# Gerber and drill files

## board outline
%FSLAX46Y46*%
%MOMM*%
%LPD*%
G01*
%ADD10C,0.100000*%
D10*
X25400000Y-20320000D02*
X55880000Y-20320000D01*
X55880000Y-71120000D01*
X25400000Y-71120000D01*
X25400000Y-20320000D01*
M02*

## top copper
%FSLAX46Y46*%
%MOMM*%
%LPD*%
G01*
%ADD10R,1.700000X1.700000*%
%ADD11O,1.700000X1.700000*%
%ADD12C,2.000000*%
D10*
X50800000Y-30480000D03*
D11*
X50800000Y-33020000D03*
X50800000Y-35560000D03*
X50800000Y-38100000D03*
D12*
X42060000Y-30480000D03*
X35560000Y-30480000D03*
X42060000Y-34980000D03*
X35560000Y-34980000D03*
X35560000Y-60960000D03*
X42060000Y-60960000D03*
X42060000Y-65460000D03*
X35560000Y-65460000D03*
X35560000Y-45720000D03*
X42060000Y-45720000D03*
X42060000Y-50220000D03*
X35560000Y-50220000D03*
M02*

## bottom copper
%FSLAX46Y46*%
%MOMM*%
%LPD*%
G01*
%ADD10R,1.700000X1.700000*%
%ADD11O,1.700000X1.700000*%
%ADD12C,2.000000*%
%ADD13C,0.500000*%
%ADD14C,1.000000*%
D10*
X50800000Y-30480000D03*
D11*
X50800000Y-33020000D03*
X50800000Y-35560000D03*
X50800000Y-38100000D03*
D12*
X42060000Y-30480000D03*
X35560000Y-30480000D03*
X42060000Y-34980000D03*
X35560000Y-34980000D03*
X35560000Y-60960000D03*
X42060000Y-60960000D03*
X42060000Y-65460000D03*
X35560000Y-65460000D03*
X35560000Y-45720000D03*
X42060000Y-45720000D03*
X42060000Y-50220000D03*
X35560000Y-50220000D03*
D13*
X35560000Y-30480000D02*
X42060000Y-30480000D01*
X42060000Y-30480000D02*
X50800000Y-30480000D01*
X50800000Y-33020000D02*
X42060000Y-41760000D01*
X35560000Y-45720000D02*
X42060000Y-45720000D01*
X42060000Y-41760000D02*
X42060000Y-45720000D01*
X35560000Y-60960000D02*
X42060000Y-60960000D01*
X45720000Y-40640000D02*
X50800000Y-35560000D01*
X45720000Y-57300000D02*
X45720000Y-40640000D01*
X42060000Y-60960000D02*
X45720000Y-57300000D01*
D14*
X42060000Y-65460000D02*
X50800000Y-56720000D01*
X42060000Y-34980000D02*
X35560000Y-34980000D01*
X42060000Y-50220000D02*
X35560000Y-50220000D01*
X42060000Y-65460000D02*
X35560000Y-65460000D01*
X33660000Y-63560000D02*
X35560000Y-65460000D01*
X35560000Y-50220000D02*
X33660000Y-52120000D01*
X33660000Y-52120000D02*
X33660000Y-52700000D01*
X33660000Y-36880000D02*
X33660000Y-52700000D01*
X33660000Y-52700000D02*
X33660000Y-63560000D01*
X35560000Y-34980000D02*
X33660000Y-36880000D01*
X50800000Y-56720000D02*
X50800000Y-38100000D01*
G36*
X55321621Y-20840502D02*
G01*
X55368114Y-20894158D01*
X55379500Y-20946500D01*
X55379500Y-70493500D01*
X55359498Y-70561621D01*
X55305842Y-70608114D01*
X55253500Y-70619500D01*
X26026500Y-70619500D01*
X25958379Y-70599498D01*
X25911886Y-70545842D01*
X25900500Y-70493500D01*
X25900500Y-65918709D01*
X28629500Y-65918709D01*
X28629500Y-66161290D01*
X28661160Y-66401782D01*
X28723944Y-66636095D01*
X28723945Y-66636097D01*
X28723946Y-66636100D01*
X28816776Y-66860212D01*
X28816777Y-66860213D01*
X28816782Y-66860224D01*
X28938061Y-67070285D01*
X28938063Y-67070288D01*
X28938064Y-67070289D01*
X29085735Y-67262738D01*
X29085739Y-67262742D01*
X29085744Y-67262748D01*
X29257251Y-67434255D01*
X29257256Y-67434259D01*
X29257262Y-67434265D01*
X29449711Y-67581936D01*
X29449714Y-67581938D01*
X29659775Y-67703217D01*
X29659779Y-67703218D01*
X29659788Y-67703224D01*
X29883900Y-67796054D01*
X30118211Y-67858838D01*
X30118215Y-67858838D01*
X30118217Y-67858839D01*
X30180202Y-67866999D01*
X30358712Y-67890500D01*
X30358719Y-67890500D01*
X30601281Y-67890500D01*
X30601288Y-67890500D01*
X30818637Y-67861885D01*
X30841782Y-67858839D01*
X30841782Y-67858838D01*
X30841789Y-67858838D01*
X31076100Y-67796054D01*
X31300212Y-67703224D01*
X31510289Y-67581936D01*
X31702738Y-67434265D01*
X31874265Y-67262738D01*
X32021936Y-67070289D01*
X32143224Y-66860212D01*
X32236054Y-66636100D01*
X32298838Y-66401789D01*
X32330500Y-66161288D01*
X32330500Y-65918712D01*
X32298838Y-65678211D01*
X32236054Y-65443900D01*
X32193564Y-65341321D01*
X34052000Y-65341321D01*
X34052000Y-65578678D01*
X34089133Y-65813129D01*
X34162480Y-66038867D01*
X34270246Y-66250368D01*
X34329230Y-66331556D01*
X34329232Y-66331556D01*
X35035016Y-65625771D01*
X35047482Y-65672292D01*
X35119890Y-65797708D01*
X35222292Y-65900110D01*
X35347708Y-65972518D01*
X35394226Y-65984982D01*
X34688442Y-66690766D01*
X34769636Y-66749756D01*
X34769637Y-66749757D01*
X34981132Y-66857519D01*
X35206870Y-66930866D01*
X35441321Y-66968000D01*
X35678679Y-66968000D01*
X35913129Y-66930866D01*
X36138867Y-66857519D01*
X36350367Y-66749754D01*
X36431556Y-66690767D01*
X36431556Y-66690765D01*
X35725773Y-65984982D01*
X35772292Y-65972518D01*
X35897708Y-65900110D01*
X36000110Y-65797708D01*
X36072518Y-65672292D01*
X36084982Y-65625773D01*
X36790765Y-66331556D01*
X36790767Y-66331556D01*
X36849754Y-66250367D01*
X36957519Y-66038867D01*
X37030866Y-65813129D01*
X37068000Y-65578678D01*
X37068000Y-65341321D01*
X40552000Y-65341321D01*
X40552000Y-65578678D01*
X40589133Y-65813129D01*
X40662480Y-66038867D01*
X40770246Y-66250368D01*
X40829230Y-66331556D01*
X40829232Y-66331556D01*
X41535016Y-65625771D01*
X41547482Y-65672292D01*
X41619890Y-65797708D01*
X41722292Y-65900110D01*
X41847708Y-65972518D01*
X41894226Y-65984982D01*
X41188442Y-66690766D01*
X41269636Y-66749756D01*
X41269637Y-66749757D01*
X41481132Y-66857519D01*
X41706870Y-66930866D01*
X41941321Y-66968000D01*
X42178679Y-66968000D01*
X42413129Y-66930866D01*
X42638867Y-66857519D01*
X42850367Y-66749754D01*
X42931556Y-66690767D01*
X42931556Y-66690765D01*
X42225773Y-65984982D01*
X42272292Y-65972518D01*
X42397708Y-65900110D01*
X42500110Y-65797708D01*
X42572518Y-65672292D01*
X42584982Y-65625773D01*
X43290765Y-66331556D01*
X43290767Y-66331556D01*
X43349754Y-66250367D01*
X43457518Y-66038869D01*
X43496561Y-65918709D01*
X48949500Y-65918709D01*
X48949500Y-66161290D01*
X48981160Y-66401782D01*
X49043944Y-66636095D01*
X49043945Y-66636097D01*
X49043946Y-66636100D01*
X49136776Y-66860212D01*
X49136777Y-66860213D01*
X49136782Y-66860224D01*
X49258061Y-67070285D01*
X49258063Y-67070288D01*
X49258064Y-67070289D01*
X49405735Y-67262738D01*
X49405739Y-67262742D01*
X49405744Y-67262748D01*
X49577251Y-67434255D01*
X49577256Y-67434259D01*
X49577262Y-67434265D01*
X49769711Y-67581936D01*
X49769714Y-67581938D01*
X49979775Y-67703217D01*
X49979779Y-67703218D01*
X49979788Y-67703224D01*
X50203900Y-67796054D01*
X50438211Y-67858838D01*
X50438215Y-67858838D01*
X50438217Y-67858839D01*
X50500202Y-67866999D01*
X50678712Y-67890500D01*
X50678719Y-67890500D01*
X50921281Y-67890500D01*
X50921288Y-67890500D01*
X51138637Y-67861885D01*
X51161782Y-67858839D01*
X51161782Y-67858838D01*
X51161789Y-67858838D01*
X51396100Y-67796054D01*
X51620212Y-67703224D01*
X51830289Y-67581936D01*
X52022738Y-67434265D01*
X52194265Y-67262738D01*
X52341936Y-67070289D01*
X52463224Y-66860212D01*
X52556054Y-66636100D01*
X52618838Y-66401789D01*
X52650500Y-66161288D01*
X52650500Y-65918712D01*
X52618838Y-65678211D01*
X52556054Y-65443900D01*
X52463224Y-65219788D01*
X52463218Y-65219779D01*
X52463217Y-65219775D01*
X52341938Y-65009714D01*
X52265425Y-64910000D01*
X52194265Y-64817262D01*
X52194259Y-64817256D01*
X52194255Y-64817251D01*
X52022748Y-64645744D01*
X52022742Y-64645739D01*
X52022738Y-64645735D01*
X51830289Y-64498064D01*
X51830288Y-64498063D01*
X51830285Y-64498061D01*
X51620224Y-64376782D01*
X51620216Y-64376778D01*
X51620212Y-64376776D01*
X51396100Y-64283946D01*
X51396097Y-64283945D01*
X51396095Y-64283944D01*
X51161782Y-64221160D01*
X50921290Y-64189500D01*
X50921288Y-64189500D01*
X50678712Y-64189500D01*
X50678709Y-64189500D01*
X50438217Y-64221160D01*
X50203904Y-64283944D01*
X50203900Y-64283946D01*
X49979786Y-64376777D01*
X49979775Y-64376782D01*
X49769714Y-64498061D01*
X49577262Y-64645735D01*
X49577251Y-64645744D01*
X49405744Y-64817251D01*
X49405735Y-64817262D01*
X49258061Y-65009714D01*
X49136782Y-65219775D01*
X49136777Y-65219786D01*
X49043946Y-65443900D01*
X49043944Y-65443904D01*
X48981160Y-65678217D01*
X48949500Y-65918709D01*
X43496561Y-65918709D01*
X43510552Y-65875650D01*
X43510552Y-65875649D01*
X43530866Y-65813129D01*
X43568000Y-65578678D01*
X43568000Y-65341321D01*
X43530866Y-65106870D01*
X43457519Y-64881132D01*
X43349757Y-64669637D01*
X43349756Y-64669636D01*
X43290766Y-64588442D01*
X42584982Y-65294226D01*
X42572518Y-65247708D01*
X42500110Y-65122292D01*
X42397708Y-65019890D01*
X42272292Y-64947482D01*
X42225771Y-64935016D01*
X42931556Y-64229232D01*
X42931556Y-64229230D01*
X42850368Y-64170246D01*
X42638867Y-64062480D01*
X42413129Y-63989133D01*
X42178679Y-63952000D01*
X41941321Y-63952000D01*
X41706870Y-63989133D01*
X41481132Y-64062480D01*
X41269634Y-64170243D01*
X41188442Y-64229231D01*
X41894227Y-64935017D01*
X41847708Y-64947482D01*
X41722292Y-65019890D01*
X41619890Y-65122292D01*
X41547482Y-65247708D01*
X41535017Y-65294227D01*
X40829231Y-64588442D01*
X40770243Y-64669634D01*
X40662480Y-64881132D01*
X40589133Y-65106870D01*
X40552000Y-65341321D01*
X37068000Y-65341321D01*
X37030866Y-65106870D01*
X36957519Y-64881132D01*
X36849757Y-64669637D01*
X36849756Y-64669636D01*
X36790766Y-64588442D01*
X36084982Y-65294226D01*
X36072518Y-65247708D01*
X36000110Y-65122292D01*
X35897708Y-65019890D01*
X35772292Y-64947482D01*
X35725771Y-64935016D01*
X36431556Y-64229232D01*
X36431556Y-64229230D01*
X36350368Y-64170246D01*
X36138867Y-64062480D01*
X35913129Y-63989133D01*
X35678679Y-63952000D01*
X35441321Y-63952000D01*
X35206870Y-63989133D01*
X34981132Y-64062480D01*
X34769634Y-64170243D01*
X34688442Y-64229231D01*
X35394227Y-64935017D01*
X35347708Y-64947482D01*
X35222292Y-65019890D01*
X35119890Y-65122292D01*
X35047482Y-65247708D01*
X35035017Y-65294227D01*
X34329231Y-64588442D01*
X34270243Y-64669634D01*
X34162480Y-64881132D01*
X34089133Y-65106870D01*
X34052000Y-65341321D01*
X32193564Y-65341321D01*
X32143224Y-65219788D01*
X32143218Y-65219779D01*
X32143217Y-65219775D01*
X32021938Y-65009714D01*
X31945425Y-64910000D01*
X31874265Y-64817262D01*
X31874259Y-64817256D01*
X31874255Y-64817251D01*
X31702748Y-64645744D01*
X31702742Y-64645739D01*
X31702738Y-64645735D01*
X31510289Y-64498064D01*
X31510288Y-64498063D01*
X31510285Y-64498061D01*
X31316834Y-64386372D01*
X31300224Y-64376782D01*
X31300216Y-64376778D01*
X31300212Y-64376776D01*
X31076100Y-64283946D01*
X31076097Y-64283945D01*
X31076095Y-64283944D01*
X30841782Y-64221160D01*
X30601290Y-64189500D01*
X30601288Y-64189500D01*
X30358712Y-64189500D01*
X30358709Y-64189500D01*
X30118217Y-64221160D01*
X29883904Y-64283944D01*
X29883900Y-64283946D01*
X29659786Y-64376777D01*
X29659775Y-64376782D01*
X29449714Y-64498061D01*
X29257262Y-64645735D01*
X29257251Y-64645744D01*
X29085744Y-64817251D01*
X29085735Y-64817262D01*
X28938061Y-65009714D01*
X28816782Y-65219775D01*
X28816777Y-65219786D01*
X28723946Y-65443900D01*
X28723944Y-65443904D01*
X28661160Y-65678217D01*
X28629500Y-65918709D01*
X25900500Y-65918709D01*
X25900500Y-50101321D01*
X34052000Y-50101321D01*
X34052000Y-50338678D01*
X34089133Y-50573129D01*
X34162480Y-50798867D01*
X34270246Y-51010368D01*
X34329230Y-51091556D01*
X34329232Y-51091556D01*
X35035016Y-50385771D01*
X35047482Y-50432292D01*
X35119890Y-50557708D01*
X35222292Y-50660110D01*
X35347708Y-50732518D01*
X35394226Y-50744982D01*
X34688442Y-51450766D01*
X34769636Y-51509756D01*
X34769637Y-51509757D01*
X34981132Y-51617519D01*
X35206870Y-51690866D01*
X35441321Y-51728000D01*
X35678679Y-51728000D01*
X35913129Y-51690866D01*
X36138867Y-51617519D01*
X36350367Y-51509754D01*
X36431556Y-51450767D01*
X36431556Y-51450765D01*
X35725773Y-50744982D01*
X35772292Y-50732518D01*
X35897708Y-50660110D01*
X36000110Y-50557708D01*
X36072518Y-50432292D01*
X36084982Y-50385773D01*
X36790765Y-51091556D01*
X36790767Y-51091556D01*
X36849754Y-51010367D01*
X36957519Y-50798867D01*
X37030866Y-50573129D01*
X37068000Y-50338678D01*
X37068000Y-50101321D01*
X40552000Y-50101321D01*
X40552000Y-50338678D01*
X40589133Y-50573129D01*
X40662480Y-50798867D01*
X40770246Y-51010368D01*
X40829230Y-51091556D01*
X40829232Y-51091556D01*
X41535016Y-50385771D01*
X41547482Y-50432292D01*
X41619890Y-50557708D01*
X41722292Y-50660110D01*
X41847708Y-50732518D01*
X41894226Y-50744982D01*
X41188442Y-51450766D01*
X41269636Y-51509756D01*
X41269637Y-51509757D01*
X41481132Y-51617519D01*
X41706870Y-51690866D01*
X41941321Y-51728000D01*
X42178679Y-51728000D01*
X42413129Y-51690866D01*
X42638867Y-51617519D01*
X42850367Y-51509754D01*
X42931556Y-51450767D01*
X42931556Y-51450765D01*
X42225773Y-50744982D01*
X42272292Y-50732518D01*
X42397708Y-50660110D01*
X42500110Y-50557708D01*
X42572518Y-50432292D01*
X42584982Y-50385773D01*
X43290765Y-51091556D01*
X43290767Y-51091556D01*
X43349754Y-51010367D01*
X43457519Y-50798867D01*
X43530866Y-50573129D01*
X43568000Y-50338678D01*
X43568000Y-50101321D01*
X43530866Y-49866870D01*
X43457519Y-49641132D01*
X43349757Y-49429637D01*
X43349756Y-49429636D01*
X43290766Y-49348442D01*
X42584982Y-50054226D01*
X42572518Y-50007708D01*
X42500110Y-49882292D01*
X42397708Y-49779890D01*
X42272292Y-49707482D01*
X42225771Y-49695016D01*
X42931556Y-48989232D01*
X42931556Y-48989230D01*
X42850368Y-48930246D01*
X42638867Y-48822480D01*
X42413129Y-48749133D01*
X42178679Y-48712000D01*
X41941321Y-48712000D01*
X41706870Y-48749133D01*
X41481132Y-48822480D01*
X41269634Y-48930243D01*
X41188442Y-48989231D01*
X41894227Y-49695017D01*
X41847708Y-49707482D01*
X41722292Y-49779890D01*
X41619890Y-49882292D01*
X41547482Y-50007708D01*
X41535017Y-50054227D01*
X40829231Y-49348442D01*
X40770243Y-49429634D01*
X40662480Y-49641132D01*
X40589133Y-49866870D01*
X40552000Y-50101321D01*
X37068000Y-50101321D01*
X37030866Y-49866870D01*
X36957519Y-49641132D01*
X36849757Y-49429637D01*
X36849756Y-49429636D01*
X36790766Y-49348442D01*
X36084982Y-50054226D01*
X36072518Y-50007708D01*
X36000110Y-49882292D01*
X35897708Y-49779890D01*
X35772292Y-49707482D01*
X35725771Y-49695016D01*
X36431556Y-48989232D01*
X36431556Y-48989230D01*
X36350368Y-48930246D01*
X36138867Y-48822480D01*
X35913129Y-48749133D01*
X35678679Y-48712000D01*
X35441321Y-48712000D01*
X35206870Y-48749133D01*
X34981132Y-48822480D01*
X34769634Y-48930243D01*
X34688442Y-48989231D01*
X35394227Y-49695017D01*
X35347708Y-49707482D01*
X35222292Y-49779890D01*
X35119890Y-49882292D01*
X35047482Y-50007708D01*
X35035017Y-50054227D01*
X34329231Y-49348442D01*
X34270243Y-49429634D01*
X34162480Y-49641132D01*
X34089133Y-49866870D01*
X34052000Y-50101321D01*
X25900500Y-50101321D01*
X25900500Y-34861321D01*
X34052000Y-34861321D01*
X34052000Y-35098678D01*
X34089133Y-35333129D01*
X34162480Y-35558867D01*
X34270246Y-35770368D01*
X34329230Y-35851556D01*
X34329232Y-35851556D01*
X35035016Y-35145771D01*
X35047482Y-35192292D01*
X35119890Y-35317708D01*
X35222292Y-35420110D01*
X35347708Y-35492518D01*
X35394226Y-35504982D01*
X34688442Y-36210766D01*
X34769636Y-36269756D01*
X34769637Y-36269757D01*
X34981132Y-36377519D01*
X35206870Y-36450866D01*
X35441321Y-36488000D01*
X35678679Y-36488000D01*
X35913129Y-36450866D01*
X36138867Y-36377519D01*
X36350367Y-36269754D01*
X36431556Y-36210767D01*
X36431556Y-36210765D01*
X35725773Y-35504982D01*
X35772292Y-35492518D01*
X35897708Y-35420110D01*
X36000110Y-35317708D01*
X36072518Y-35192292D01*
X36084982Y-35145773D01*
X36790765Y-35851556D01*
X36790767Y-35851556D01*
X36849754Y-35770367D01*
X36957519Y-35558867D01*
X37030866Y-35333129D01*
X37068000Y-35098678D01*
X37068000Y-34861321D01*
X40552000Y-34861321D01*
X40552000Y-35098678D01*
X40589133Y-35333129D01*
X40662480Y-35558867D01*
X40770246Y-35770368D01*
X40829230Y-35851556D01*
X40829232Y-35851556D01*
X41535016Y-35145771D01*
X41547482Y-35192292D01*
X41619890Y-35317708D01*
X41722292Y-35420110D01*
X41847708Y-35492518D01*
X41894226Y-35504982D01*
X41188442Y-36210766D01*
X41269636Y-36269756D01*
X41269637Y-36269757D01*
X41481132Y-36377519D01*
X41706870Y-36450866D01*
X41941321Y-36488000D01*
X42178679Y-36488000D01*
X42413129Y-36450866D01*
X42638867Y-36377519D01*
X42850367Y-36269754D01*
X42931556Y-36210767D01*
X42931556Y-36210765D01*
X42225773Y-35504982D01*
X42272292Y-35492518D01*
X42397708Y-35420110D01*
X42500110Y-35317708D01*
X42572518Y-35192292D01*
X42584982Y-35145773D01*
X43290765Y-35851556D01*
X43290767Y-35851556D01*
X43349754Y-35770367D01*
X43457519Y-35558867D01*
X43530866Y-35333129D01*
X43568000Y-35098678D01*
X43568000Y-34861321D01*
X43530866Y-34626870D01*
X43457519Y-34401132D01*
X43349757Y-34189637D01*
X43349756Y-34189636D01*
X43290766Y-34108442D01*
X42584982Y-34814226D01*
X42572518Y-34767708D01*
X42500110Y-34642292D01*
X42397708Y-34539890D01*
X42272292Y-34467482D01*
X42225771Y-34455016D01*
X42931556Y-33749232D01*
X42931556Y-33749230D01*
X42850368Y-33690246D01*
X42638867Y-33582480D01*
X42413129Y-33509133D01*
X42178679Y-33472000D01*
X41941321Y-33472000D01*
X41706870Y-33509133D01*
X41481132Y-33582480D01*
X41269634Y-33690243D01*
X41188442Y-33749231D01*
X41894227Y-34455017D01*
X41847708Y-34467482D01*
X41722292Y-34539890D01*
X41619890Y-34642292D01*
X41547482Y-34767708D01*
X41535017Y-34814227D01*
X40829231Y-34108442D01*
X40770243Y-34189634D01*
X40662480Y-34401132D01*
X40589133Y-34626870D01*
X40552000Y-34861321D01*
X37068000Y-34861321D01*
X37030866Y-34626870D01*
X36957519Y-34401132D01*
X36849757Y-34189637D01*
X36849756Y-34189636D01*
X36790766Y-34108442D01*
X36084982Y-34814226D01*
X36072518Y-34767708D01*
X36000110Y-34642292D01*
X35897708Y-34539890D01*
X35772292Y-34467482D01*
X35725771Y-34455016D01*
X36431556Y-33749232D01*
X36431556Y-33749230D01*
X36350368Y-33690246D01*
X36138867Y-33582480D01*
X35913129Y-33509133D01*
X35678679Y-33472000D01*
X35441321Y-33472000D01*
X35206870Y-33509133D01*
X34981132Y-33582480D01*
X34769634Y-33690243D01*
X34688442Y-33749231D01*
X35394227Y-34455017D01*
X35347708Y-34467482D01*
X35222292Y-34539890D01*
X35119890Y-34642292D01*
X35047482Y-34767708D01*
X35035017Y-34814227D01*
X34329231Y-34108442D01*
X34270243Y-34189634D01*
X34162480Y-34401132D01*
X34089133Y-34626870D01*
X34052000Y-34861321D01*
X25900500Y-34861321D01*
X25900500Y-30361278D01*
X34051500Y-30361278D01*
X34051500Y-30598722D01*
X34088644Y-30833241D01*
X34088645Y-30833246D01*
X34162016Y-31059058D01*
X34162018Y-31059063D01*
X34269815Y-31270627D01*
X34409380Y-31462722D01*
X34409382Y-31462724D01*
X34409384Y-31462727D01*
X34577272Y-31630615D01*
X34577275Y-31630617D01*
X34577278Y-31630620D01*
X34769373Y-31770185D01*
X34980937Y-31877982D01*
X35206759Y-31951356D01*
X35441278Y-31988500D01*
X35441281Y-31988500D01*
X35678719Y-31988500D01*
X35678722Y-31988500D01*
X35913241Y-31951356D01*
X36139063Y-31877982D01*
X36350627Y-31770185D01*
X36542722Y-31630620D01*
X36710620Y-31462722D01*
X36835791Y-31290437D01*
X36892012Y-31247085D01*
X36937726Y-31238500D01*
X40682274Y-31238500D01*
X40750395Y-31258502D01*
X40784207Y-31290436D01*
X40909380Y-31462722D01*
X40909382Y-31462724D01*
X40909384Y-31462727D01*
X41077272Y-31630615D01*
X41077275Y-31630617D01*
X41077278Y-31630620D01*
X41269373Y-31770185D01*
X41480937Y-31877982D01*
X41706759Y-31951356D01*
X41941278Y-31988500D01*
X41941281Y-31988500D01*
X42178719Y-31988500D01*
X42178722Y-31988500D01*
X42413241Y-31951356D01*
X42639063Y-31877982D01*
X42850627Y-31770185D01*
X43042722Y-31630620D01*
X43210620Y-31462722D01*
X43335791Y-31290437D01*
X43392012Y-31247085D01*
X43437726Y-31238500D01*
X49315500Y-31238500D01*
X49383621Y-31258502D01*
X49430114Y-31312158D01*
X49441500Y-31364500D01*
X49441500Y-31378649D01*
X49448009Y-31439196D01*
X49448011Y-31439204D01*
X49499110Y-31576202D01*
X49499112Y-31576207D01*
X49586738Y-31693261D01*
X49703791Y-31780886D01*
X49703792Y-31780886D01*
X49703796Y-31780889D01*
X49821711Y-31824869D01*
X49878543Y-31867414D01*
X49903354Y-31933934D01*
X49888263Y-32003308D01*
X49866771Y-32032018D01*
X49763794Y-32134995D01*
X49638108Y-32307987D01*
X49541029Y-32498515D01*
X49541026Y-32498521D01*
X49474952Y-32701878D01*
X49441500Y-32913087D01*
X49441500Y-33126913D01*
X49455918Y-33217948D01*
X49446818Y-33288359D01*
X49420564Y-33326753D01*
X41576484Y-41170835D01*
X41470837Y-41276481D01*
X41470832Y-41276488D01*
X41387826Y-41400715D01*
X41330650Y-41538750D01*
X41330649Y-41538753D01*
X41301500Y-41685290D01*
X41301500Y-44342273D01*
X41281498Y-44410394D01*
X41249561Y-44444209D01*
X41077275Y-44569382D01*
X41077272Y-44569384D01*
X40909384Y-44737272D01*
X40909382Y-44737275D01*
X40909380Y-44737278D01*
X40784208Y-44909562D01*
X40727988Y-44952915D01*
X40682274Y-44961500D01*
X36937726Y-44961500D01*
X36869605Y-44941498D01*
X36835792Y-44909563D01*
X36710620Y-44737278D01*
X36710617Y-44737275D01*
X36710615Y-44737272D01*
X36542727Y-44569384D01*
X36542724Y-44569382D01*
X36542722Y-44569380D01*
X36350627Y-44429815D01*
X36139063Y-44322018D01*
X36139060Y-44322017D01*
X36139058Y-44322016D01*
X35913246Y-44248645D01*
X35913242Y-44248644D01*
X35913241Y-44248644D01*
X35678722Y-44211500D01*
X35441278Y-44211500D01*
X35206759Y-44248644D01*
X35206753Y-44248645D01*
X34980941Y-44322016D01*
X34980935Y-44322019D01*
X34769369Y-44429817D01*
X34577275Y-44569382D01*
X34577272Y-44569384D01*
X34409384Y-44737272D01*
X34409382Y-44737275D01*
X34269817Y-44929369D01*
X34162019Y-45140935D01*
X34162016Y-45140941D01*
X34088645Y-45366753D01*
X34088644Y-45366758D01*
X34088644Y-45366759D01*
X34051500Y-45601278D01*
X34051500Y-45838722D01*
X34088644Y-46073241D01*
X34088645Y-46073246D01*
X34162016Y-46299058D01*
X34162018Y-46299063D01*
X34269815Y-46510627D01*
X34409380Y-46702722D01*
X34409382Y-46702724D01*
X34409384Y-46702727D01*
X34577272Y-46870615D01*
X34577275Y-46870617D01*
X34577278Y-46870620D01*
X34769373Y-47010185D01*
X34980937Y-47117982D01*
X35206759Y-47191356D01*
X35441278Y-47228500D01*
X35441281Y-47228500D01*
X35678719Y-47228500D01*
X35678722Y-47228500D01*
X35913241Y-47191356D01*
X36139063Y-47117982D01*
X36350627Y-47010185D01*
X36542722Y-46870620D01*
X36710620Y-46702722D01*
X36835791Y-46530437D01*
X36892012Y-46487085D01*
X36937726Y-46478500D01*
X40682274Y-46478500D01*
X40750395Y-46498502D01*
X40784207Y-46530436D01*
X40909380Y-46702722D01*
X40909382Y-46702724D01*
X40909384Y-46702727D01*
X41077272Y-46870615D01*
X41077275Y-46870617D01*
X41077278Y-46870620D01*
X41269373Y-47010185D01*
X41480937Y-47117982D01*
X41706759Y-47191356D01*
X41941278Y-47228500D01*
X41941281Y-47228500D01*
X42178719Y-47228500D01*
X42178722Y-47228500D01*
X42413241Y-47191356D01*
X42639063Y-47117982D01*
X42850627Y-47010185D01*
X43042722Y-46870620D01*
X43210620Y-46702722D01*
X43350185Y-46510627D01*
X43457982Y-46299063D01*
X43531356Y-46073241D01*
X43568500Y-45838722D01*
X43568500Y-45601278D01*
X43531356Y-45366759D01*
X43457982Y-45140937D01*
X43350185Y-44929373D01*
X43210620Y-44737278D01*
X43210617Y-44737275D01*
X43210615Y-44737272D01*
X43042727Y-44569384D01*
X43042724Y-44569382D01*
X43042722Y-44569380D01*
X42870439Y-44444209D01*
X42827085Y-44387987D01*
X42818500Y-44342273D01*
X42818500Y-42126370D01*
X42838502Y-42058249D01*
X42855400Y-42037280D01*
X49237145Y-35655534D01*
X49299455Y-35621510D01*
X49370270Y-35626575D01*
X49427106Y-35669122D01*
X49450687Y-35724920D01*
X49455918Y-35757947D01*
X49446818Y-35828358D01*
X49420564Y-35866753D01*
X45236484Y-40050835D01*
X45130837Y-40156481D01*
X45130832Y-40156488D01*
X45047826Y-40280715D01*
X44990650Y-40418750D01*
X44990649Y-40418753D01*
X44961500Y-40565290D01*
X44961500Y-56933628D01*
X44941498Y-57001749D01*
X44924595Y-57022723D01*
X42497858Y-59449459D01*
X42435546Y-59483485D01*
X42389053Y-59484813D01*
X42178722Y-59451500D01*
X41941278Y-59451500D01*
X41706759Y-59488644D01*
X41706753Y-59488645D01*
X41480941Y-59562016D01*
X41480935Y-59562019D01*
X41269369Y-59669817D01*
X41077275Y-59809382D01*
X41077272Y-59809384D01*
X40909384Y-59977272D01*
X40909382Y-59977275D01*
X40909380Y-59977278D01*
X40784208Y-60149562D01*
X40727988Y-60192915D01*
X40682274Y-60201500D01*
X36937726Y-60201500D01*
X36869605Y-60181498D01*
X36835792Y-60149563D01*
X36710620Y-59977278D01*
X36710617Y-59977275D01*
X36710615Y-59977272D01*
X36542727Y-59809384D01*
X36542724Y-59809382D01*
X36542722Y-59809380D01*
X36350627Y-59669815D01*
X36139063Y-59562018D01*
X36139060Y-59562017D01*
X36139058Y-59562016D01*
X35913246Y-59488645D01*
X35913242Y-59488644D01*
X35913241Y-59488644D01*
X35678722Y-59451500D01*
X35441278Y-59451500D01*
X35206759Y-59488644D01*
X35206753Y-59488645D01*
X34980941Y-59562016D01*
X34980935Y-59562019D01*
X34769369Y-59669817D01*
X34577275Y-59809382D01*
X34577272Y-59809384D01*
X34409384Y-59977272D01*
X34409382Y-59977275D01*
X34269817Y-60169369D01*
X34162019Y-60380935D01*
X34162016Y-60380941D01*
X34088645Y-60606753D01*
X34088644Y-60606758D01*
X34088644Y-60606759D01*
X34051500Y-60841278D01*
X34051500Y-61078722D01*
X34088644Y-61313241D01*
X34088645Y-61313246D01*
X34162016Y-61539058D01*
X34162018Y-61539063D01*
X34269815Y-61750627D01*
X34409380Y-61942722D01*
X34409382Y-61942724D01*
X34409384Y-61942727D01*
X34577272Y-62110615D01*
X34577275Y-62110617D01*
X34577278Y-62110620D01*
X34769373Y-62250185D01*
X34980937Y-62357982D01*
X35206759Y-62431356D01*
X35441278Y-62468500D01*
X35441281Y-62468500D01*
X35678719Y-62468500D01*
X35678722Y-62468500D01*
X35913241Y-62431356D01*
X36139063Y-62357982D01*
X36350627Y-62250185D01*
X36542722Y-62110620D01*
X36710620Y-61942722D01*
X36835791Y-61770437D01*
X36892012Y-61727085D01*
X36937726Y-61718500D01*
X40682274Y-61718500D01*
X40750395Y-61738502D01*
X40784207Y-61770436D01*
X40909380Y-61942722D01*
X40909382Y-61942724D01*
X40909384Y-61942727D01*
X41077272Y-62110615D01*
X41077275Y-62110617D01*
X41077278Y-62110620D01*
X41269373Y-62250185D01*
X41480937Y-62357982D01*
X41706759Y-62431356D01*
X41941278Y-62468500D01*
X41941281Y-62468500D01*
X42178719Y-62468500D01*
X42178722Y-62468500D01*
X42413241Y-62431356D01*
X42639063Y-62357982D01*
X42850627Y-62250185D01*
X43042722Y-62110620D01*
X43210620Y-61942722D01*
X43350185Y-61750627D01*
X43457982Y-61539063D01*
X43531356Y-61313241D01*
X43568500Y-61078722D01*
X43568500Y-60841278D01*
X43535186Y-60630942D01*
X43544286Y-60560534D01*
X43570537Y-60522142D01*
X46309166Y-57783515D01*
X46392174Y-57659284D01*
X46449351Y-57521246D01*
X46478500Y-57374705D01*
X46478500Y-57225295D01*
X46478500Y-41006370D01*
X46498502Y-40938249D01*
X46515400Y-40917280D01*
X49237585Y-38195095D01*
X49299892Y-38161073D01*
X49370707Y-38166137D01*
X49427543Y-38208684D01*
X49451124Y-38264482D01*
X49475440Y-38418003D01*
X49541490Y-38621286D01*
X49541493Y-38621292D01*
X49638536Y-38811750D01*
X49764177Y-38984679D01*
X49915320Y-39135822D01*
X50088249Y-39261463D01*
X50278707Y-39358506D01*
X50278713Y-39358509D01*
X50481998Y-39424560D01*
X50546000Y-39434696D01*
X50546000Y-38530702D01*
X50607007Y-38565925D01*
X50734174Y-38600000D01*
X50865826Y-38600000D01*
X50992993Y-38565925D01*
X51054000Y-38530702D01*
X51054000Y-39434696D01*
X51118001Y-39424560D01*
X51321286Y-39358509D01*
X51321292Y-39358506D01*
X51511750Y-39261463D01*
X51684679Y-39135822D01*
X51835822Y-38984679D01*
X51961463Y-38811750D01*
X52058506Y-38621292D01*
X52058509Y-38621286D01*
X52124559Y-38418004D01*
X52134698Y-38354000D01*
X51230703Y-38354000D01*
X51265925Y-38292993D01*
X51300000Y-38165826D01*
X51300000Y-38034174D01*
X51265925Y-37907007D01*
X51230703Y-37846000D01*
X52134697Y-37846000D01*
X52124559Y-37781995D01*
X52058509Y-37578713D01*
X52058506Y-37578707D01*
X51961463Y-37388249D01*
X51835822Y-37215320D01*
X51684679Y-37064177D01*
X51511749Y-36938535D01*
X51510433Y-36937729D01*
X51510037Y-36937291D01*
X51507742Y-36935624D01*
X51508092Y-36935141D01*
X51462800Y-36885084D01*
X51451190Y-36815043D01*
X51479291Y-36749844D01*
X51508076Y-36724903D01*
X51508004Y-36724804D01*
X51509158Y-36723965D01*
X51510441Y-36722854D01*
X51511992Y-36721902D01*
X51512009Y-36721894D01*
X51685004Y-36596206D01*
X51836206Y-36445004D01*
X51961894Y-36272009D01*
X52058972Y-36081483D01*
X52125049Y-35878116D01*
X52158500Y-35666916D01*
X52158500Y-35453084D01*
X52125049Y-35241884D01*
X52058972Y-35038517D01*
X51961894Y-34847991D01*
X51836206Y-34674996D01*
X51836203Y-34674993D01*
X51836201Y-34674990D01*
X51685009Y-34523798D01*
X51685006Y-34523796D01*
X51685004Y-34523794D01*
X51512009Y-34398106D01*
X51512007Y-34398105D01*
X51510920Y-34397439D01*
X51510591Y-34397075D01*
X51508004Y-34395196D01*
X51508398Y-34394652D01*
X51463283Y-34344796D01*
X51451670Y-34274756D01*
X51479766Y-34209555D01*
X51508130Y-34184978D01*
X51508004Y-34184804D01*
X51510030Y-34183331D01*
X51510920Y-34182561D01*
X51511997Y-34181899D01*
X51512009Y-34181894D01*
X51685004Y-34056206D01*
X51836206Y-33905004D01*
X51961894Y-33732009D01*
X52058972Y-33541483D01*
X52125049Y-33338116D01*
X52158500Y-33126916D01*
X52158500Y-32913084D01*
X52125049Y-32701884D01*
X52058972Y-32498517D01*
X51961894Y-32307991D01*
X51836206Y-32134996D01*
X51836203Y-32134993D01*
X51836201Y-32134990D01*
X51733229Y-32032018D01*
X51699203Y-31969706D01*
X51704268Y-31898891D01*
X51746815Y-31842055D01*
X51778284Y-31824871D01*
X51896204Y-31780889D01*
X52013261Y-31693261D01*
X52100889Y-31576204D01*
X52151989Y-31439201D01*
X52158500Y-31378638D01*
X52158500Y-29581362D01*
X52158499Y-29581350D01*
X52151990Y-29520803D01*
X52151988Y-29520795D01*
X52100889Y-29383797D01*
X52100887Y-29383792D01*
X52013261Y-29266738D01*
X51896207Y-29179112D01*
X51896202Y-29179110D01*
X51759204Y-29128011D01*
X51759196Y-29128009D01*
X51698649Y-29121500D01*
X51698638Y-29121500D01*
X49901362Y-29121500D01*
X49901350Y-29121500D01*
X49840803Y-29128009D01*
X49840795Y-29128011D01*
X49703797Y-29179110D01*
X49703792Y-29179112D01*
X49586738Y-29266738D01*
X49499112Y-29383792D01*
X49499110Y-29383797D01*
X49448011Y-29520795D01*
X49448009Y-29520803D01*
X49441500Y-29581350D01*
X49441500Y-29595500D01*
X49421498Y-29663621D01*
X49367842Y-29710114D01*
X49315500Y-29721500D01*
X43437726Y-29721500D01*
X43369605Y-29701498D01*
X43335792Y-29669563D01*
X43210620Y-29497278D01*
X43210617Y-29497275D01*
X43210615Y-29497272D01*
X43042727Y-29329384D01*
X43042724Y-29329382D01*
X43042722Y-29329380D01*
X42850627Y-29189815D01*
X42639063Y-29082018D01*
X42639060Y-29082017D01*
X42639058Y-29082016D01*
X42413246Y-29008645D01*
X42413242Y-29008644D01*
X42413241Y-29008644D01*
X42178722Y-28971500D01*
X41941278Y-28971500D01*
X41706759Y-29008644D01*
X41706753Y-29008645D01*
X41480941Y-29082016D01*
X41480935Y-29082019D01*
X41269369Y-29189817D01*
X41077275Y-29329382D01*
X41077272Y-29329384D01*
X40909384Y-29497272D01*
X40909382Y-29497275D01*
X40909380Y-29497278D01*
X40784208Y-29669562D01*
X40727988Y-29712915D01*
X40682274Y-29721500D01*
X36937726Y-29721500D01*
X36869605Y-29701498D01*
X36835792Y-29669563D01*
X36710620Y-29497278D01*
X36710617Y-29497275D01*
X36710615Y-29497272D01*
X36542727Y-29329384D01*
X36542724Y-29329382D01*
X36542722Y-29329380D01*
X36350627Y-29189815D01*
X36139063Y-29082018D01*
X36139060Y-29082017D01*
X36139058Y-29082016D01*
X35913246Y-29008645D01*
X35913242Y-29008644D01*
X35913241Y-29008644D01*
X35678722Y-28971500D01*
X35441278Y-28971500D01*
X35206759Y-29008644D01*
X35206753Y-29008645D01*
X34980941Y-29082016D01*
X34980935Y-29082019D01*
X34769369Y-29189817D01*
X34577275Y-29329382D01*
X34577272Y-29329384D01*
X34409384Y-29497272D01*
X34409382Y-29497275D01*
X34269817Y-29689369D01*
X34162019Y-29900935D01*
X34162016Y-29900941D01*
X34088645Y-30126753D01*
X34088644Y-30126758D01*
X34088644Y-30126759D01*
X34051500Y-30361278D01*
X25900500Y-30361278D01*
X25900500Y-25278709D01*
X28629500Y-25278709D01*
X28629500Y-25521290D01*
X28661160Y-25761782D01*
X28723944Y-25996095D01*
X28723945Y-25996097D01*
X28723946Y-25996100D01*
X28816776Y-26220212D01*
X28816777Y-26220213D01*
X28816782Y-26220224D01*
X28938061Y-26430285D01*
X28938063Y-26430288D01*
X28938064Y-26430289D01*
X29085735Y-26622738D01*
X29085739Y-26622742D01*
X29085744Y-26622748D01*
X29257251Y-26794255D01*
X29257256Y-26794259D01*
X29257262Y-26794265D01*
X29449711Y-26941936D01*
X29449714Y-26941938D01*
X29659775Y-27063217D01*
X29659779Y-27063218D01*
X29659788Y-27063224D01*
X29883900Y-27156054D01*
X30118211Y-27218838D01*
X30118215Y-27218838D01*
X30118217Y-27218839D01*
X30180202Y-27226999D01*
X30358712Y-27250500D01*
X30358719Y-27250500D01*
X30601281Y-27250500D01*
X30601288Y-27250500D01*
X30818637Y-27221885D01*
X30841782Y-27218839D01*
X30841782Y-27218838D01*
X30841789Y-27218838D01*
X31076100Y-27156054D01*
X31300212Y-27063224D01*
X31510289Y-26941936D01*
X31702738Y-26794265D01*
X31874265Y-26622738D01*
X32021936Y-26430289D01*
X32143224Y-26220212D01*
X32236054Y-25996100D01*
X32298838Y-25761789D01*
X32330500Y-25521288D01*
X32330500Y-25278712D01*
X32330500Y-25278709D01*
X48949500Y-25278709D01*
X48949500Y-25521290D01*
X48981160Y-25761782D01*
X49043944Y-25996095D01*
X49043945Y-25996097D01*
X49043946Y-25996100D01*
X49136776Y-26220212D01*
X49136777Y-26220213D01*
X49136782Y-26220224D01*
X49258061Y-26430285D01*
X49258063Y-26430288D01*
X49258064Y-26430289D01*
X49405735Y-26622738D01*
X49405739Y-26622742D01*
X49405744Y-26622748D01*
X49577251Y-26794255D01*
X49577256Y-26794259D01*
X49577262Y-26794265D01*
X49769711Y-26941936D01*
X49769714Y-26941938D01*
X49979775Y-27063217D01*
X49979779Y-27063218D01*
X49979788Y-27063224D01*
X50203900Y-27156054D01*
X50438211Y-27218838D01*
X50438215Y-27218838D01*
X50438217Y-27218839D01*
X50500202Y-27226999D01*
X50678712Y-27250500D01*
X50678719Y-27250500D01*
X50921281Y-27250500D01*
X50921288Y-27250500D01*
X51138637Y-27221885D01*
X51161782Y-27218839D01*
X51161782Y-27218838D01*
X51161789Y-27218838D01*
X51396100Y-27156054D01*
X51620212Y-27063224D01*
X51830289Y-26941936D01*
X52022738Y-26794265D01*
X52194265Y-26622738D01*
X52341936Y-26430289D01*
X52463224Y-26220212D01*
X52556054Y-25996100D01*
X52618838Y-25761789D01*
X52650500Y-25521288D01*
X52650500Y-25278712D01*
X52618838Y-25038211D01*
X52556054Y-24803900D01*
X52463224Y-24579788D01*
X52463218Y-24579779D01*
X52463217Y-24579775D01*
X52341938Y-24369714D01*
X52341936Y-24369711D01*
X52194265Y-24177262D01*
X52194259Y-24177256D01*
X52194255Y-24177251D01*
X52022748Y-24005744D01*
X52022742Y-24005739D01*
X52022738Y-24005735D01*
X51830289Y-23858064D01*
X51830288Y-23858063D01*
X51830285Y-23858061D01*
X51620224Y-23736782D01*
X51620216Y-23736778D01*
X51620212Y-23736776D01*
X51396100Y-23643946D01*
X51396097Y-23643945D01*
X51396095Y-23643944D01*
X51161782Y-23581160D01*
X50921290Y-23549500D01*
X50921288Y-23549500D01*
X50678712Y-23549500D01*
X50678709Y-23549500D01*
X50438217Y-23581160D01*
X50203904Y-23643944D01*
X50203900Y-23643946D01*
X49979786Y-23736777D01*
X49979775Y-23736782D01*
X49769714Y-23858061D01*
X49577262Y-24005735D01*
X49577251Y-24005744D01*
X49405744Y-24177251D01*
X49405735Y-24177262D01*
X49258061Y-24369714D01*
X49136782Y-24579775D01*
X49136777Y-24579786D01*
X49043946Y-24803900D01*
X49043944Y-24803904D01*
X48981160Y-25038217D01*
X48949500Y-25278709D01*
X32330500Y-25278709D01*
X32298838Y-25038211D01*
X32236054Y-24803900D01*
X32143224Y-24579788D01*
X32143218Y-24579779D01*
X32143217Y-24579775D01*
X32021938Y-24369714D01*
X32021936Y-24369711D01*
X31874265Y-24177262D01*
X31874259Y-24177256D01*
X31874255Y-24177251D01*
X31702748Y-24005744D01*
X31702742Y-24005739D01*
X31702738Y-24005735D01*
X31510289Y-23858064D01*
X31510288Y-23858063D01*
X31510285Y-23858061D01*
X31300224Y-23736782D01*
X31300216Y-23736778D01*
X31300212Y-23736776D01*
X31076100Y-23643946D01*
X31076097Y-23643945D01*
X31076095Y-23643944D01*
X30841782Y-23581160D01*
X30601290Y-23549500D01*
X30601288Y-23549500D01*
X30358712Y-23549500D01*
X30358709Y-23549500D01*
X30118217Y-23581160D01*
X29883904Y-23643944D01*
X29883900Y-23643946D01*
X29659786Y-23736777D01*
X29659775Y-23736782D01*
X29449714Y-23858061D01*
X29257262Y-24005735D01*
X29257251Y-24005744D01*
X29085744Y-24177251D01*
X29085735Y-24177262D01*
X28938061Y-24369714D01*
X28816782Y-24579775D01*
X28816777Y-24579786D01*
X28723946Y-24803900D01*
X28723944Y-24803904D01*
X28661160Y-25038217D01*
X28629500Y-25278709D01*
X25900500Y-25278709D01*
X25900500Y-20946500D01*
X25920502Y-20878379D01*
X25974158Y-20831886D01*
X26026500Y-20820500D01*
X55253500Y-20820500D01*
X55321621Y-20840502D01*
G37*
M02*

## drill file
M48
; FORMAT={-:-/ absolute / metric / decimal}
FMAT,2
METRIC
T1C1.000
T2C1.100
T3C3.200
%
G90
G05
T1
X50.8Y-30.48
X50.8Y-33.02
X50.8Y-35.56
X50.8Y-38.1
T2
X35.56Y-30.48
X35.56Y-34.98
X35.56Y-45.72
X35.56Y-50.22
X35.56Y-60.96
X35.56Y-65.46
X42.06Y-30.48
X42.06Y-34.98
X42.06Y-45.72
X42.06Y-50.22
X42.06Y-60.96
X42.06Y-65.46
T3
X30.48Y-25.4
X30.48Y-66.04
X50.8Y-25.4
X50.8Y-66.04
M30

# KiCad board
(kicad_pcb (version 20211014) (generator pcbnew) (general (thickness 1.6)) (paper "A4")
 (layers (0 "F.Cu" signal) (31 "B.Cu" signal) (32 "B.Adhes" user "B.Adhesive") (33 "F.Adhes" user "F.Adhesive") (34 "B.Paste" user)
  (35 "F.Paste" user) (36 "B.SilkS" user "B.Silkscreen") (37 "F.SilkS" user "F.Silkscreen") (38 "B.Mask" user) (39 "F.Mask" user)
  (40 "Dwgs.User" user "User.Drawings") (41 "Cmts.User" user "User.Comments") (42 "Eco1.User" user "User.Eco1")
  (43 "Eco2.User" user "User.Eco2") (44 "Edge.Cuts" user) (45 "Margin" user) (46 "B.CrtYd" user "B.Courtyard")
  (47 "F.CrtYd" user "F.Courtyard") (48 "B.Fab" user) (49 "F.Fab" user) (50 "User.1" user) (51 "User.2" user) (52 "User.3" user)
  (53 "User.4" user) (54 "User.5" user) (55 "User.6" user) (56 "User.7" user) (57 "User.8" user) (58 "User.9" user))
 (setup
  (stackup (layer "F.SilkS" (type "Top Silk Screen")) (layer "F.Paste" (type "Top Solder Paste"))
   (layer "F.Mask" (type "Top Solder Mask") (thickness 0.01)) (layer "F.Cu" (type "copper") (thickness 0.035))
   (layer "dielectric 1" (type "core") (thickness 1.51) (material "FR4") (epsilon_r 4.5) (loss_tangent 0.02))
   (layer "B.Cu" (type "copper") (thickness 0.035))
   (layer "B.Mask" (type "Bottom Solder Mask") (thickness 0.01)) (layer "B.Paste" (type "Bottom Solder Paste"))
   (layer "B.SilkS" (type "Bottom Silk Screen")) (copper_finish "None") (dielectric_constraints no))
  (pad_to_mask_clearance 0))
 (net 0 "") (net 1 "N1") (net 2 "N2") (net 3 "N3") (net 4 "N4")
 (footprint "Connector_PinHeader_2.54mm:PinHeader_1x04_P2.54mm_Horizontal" (layer "F.Cu") (at 50.8 30.48)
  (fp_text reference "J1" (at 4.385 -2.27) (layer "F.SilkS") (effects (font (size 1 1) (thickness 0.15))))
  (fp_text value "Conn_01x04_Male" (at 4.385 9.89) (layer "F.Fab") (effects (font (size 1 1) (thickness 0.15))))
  (pad "1" thru_hole rect (at 0 0) (size 1.7 1.7) (drill 1) (layers *.Cu *.Mask) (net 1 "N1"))
  (pad "2" thru_hole oval (at 0 2.54) (size 1.7 1.7) (drill 1) (layers *.Cu *.Mask) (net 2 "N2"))
  (pad "3" thru_hole oval (at 0 5.08) (size 1.7 1.7) (drill 1) (layers *.Cu *.Mask) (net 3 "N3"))
  (pad "4" thru_hole oval (at 0 7.62) (size 1.7 1.7) (drill 1) (layers *.Cu *.Mask) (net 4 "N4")))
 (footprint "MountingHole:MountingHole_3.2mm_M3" (layer "F.Cu") (at 30.48 66.04)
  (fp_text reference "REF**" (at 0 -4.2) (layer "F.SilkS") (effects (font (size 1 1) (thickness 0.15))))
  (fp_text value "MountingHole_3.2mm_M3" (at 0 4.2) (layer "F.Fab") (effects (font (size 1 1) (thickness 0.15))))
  (pad "" np_thru_hole circle (at 0 0) (size 3.2 3.2) (drill 3.2) (layers *.Cu *.Mask)))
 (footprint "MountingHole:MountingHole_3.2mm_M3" (layer "F.Cu") (at 50.8 66.04)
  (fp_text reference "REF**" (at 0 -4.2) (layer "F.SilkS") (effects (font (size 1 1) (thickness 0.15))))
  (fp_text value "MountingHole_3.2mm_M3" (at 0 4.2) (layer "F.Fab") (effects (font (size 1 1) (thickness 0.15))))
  (pad "" np_thru_hole circle (at 0 0) (size 3.2 3.2) (drill 3.2) (layers *.Cu *.Mask)))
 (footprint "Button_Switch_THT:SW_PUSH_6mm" (layer "F.Cu") (at 35.56 30.48)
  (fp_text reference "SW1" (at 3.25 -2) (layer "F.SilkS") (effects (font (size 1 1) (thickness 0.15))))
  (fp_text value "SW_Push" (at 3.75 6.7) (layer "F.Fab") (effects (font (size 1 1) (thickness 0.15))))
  (pad "1" thru_hole circle (at 6.5 0 90) (size 2 2) (drill 1.1) (layers *.Cu *.Mask) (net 1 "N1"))
  (pad "1" thru_hole circle (at 0 0 90) (size 2 2) (drill 1.1) (layers *.Cu *.Mask) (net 1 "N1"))
  (pad "2" thru_hole circle (at 6.5 4.5 90) (size 2 2) (drill 1.1) (layers *.Cu *.Mask) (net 4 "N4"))
  (pad "2" thru_hole circle (at 0 4.5 90) (size 2 2) (drill 1.1) (layers *.Cu *.Mask) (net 4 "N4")))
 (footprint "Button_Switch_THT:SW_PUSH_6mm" (layer "F.Cu") (at 35.56 60.96)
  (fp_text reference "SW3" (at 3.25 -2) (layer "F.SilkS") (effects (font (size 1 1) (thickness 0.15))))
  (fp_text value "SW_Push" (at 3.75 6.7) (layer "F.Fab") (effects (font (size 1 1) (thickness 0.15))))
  (pad "1" thru_hole circle (at 0 0 90) (size 2 2) (drill 1.1) (layers *.Cu *.Mask) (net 3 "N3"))
  (pad "1" thru_hole circle (at 6.5 0 90) (size 2 2) (drill 1.1) (layers *.Cu *.Mask) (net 3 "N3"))
  (pad "2" thru_hole circle (at 6.5 4.5 90) (size 2 2) (drill 1.1) (layers *.Cu *.Mask) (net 4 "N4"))
  (pad "2" thru_hole circle (at 0 4.5 90) (size 2 2) (drill 1.1) (layers *.Cu *.Mask) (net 4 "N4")))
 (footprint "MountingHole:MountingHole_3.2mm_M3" (layer "F.Cu") (at 30.48 25.4)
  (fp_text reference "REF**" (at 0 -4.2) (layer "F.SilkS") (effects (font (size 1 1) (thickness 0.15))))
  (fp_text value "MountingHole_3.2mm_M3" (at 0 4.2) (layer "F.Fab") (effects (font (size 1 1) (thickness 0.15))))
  (pad "" np_thru_hole circle (at 0 0) (size 3.2 3.2) (drill 3.2) (layers *.Cu *.Mask)))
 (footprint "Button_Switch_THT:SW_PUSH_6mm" (layer "F.Cu") (at 35.56 45.72)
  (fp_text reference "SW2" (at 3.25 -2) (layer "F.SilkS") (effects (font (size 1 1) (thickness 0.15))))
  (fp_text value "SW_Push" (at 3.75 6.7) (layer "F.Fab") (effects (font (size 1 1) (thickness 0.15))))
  (pad "1" thru_hole circle (at 0 0 90) (size 2 2) (drill 1.1) (layers *.Cu *.Mask) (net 2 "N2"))
  (pad "1" thru_hole circle (at 6.5 0 90) (size 2 2) (drill 1.1) (layers *.Cu *.Mask) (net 2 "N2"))
  (pad "2" thru_hole circle (at 6.5 4.5 90) (size 2 2) (drill 1.1) (layers *.Cu *.Mask) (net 4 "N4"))
  (pad "2" thru_hole circle (at 0 4.5 90) (size 2 2) (drill 1.1) (layers *.Cu *.Mask) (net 4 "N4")))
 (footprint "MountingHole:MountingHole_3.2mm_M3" (layer "F.Cu") (at 50.8 25.4)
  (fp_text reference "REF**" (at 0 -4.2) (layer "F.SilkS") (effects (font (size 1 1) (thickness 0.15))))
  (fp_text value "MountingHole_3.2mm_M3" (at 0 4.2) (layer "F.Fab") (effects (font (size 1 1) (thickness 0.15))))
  (pad "" np_thru_hole circle (at 0 0) (size 3.2 3.2) (drill 3.2) (layers *.Cu *.Mask)))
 (gr_rect (start 25.4 20.32) (end 55.88 71.12) (layer "Edge.Cuts") (width 0.1) (fill none))
 (segment (start 35.56 30.48) (end 42.06 30.48) (width 0.5) (layer "B.Cu") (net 1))
 (segment (start 42.06 30.48) (end 50.8 30.48) (width 0.5) (layer "B.Cu") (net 1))
 (segment (start 50.8 33.02) (end 42.06 41.76) (width 0.5) (layer "B.Cu") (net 2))
 (segment (start 35.56 45.72) (end 42.06 45.72) (width 0.5) (layer "B.Cu") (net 2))
 (segment (start 42.06 41.76) (end 42.06 45.72) (width 0.5) (layer "B.Cu") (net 2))
 (segment (start 35.56 60.96) (end 42.06 60.96) (width 0.5) (layer "B.Cu") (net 3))
 (segment (start 45.72 40.64) (end 50.8 35.56) (width 0.5) (layer "B.Cu") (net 3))
 (segment (start 45.72 57.3) (end 45.72 40.64) (width 0.5) (layer "B.Cu") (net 3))
 (segment (start 42.06 60.96) (end 45.72 57.3) (width 0.5) (layer "B.Cu") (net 3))
 (segment (start 42.06 65.46) (end 50.8 56.72) (width 1) (layer "B.Cu") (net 4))
 (segment (start 42.06 34.98) (end 35.56 34.98) (width 1) (layer "B.Cu") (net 4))
 (segment (start 42.06 50.22) (end 35.56 50.22) (width 1) (layer "B.Cu") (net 4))
 (segment (start 42.06 65.46) (end 35.56 65.46) (width 1) (layer "B.Cu") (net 4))
 (segment (start 33.66 63.56) (end 35.56 65.46) (width 1) (layer "B.Cu") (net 4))
 (segment (start 35.56 50.22) (end 33.66 52.12) (width 1) (layer "B.Cu") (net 4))
 (segment (start 33.66 52.12) (end 33.66 52.7) (width 1) (layer "B.Cu") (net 4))
 (segment (start 33.66 36.88) (end 33.66 52.7) (width 1) (layer "B.Cu") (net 4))
 (segment (start 33.66 52.7) (end 33.66 63.56) (width 1) (layer "B.Cu") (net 4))
 (segment (start 35.56 34.98) (end 33.66 36.88) (width 1) (layer "B.Cu") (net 4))
 (segment (start 50.8 56.72) (end 50.8 38.1) (width 1) (layer "B.Cu") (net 4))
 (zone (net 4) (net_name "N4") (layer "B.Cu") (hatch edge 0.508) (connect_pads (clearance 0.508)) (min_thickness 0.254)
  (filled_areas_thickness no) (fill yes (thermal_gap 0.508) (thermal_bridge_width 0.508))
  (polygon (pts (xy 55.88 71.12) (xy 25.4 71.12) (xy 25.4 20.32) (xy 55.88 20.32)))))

